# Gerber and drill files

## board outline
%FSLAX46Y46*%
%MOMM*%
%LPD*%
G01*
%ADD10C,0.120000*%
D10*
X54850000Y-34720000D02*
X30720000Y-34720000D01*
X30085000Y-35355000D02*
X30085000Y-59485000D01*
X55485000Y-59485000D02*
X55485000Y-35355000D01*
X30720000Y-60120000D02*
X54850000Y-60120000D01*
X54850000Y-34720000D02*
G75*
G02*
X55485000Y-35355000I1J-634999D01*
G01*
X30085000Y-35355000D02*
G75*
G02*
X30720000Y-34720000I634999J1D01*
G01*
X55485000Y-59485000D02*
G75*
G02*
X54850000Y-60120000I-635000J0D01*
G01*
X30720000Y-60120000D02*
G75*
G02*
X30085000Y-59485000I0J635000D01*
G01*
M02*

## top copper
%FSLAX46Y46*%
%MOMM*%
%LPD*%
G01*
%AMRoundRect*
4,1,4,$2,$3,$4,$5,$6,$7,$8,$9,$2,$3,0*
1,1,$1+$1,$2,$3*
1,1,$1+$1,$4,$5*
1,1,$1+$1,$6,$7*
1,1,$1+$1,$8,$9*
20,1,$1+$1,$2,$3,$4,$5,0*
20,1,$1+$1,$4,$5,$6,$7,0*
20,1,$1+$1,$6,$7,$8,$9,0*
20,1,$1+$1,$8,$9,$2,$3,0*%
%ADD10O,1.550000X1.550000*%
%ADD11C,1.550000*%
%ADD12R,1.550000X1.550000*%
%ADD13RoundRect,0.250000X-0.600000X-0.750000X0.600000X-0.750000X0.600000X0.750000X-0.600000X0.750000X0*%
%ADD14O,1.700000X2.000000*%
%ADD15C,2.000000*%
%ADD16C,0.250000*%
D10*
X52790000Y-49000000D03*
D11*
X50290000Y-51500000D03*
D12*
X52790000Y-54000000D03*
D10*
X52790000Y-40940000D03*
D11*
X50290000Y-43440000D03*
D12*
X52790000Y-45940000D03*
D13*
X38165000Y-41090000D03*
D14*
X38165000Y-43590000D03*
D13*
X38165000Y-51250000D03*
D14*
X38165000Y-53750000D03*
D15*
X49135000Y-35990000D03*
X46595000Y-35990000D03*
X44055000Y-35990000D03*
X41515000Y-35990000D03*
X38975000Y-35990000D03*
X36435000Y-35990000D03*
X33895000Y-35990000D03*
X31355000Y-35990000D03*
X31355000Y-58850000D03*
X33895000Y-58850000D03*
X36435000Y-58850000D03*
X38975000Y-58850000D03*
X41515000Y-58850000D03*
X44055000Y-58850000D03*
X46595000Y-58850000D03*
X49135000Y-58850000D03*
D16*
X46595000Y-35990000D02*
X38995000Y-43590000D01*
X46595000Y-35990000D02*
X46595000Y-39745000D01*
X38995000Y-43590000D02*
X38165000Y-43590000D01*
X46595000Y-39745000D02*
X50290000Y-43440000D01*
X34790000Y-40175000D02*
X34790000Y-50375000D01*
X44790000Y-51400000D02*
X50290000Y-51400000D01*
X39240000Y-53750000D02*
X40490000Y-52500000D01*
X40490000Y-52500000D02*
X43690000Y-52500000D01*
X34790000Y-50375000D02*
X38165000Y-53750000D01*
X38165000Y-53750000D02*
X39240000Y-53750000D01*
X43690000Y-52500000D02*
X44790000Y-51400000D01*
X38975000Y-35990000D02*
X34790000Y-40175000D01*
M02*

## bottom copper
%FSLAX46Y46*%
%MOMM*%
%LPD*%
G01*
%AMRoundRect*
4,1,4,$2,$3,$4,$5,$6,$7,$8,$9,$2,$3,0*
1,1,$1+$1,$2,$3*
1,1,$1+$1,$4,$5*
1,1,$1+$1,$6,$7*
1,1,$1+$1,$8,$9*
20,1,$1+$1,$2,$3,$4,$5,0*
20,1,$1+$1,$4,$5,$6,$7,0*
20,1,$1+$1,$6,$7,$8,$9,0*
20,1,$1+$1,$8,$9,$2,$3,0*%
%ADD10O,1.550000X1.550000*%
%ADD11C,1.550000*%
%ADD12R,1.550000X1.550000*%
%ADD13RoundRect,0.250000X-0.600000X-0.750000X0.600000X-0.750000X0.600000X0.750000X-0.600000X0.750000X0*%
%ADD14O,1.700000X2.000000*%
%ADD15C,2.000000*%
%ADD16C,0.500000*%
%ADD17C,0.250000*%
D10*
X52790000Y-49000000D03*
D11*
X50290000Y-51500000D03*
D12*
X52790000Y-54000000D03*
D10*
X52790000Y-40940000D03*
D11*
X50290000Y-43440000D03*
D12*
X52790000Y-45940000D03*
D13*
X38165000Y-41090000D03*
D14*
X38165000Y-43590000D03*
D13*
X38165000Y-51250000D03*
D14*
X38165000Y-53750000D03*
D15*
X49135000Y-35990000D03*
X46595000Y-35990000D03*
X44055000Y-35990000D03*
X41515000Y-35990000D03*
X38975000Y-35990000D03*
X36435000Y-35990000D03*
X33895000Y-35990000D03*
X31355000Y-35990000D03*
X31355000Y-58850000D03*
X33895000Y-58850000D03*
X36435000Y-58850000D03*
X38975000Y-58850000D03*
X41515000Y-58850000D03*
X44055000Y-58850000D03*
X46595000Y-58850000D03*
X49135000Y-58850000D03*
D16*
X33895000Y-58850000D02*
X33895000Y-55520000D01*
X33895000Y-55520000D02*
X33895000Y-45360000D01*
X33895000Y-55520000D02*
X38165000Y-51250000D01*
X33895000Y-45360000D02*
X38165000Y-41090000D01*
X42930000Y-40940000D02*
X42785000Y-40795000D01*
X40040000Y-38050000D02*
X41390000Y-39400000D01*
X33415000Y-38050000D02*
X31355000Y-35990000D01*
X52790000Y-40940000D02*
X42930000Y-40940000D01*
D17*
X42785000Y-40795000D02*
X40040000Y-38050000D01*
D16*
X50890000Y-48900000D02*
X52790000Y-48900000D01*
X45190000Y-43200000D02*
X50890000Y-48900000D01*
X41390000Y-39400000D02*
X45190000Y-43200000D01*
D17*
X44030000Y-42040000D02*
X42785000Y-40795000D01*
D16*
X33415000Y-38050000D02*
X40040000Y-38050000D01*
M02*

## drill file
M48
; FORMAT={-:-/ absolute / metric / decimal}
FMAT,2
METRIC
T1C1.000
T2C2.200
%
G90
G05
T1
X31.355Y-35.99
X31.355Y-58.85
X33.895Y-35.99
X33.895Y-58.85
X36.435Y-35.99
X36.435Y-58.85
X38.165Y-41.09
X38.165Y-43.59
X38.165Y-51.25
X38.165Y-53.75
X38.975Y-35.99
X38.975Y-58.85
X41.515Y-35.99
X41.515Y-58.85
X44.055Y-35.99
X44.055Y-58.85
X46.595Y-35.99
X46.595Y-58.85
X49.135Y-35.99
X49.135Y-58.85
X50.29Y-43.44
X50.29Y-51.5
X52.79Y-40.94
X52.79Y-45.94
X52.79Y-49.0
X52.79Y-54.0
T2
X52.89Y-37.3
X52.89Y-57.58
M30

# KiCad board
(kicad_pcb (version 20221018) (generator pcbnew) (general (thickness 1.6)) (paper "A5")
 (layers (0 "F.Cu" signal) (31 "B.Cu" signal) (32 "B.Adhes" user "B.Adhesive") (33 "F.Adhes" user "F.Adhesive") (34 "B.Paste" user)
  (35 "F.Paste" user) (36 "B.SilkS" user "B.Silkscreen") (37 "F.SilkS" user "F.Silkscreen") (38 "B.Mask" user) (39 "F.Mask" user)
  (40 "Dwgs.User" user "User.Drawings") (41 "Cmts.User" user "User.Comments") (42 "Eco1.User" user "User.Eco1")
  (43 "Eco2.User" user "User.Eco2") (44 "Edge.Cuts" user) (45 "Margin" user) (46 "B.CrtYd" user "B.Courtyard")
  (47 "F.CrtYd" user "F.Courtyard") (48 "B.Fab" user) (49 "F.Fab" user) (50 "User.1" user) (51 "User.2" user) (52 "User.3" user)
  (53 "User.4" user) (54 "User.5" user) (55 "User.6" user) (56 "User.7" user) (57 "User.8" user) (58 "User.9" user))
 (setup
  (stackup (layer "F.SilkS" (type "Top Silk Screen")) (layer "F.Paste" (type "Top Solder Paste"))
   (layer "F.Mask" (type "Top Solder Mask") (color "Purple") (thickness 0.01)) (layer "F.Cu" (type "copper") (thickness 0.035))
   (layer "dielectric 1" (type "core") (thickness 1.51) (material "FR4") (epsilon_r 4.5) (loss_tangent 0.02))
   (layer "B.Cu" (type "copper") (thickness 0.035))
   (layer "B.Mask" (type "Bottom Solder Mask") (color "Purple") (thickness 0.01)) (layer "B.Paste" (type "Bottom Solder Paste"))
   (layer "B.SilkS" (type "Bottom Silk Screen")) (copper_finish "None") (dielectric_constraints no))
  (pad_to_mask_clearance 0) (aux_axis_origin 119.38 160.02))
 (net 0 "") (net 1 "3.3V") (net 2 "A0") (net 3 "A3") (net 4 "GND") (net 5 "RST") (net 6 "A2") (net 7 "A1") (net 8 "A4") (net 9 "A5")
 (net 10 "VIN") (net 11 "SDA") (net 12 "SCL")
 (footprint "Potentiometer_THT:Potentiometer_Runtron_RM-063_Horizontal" (layer "F.Cu") (at 52.79 49 -90)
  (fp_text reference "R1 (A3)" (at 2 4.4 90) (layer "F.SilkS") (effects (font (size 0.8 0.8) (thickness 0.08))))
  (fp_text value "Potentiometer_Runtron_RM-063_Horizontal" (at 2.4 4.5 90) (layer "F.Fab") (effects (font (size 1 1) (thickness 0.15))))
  (pad "1" thru_hole oval (at 0 0 270) (size 1.55 1.55) (drill 1) (layers "*.Cu" "*.Mask") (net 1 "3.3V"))
  (pad "2" thru_hole circle (at 2.5 2.5 270) (size 1.55 1.55) (drill 1) (layers "*.Cu" "*.Mask") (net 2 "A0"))
  (pad "3" thru_hole rect (at 5 0 270) (size 1.55 1.55) (drill 1) (layers "*.Cu" "*.Mask")))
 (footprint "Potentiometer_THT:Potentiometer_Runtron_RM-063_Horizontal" (layer "F.Cu") (at 52.79 40.94 -90)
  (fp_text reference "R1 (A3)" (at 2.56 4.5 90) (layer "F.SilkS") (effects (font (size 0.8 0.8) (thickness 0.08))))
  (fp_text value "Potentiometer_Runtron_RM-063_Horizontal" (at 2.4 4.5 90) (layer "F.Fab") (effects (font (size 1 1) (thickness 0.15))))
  (pad "1" thru_hole oval (at 0 0 270) (size 1.55 1.55) (drill 1) (layers "*.Cu" "*.Mask") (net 1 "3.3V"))
  (pad "2" thru_hole circle (at 2.5 2.5 270) (size 1.55 1.55) (drill 1) (layers "*.Cu" "*.Mask") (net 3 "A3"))
  (pad "3" thru_hole rect (at 5 0 270) (size 1.55 1.55) (drill 1) (layers "*.Cu" "*.Mask")))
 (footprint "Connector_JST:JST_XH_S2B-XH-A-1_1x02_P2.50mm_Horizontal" (layer "F.Cu") (at 30.065 42.34 -90)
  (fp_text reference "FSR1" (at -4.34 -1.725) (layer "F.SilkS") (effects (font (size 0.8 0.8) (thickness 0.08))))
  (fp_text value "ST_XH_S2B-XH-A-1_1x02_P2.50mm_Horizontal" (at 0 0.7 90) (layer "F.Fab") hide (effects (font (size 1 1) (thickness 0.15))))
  (pad "1" thru_hole roundrect (at -1.25 -8.1) (size 1.7 2) (drill 1) (layers "*.Cu" "*.Mask") (roundrect_rratio 0.1470588235) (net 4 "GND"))
  (pad "2" thru_hole oval (at 1.25 -8.1) (size 1.7 2) (drill 1) (layers "*.Cu" "*.Mask") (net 3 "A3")))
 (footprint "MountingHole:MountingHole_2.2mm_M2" (layer "F.Cu") (at 52.89 57.54)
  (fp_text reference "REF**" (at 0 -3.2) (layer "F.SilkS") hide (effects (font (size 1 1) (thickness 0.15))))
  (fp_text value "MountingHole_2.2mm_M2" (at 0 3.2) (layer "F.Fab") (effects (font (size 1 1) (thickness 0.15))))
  (pad "" np_thru_hole circle (at 0 0.04) (size 2.2 2.2) (drill 2.2) (layers "*.Cu" "*.Mask")))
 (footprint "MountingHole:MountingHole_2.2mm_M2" (layer "F.Cu") (at 52.89 37.3)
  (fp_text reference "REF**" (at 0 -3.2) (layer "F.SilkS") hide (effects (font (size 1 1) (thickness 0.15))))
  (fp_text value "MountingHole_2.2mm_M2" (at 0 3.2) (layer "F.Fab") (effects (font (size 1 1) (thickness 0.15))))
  (pad "" np_thru_hole circle (at 0 0) (size 2.2 2.2) (drill 2.2) (layers "*.Cu" "*.Mask")))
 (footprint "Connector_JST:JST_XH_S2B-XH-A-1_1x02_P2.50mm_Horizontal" (layer "F.Cu") (at 30.065 52.5 -90)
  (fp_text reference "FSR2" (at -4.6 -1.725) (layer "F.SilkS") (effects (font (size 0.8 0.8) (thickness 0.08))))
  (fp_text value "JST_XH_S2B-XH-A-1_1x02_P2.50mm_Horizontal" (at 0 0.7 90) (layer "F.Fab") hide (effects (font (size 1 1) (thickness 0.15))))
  (pad "1" thru_hole roundrect (at -1.25 -8.1) (size 1.7 2) (drill 1) (layers "*.Cu" "*.Mask") (roundrect_rratio 0.1470588235) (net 4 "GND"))
  (pad "2" thru_hole oval (at 1.25 -8.1) (size 1.7 2) (drill 1) (layers "*.Cu" "*.Mask") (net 2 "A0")))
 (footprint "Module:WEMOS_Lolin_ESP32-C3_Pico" (layer "F.Cu") (at 30.085 47.42 -90)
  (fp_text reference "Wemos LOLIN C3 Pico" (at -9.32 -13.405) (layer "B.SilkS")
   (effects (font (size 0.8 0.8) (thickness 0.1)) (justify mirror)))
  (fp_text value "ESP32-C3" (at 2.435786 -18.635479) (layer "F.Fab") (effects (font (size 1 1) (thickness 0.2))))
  (fp_line (start -12.7 -24.765) (end -12.7 -0.635) (stroke (width 0.12) (type solid)) (layer "Edge.Cuts"))
  (fp_line (start -12.065 0) (end 12.065 0) (stroke (width 0.12) (type solid)) (layer "Edge.Cuts"))
  (fp_line (start 12.065 -25.4) (end -12.065 -25.4) (stroke (width 0.12) (type solid)) (layer "Edge.Cuts"))
  (fp_line (start 12.7 -0.635) (end 12.7 -24.765) (stroke (width 0.12) (type solid)) (layer "Edge.Cuts"))
  (fp_arc (start -12.7 -24.765) (mid -12.514013 -25.214013) (end -12.065 -25.4) (stroke (width 0.12) (type solid)) (layer "Edge.Cuts"))
  (fp_arc (start -12.065 0) (mid -12.514013 -0.185987) (end -12.7 -0.635) (stroke (width 0.12) (type solid)) (layer "Edge.Cuts"))
  (fp_arc (start 12.065 -25.4) (mid 12.514013 -25.214013) (end 12.7 -24.765) (stroke (width 0.12) (type solid)) (layer "Edge.Cuts"))
  (fp_arc (start 12.7 -0.635) (mid 12.514013 -0.185987) (end 12.065 0) (stroke (width 0.12) (type solid)) (layer "Edge.Cuts"))
  (pad "1" thru_hole circle (at -11.43 -19.05 270) (size 2 2) (drill 1) (layers "*.Cu" "*.Mask") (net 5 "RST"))
  (pad "2" thru_hole circle (at -11.43 -16.51 270) (size 2 2) (drill 1) (layers "*.Cu" "*.Mask") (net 3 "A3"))
  (pad "3" thru_hole circle (at -11.43 -13.97 270) (size 2 2) (drill 1) (layers "*.Cu" "*.Mask") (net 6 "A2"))
  (pad "4" thru_hole circle (at -11.43 -11.43 270) (size 2 2) (drill 1) (layers "*.Cu" "*.Mask") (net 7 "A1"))
  (pad "5" thru_hole circle (at -11.43 -8.89 270) (size 2 2) (drill 1) (layers "*.Cu" "*.Mask") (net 2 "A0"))
  (pad "6" thru_hole circle (at -11.43 -6.35 270) (size 2 2) (drill 1) (layers "*.Cu" "*.Mask") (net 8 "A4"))
  (pad "7" thru_hole circle (at -11.43 -3.81 270) (size 2 2) (drill 1) (layers "*.Cu" "*.Mask") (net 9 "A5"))
  (pad "8" thru_hole circle (at -11.43 -1.27 270) (size 2 2) (drill 1) (layers "*.Cu" "*.Mask") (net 1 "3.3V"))
  (pad "9" thru_hole circle (at 11.43 -1.27 270) (size 2 2) (drill 1) (layers "*.Cu" "*.Mask") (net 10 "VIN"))
  (pad "10" thru_hole circle (at 11.43 -3.81 270) (size 2 2) (drill 1) (layers "*.Cu" "*.Mask") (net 4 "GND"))
  (pad "11" thru_hole circle (at 11.43 -6.35 270) (size 2 2) (drill 1) (layers "*.Cu" "*.Mask"))
  (pad "12" thru_hole circle (at 11.43 -8.89 270) (size 2 2) (drill 1) (layers "*.Cu" "*.Mask"))
  (pad "13" thru_hole circle (at 11.43 -11.43 270) (size 2 2) (drill 1) (layers "*.Cu" "*.Mask") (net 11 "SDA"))
  (pad "14" thru_hole circle (at 11.43 -13.97 270) (size 2 2) (drill 1) (layers "*.Cu" "*.Mask") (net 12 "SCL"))
  (pad "15" thru_hole circle (at 11.43 -16.51 270) (size 2 2) (drill 1) (layers "*.Cu" "*.Mask"))
  (pad "16" thru_hole circle (at 11.43 -19.05 270) (size 2 2) (drill 1) (layers "*.Cu" "*.Mask")))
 (segment (start 33.895 58.85) (end 33.895 55.52) (width 0.5) (layer "B.Cu") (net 4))
 (segment (start 33.895 55.52) (end 33.895 45.36) (width 0.5) (layer "B.Cu") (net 4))
 (segment (start 33.895 55.52) (end 38.165 51.25) (width 0.5) (layer "B.Cu") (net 4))
 (segment (start 33.895 45.36) (end 38.165 41.09) (width 0.5) (layer "B.Cu") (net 4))
 (segment (start 42.93 40.94) (end 42.785 40.795) (width 0.5) (layer "B.Cu") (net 1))
 (segment (start 40.04 38.05) (end 41.39 39.4) (width 0.5) (layer "B.Cu") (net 1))
 (segment (start 33.415 38.05) (end 31.355 35.99) (width 0.5) (layer "B.Cu") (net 1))
 (segment (start 52.79 40.94) (end 42.93 40.94) (width 0.5) (layer "B.Cu") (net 1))
 (segment (start 42.785 40.795) (end 40.04 38.05) (width 0.25) (layer "B.Cu") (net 1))
 (segment (start 50.89 48.9) (end 52.79 48.9) (width 0.5) (layer "B.Cu") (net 1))
 (segment (start 45.19 43.2) (end 50.89 48.9) (width 0.5) (layer "B.Cu") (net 1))
 (segment (start 41.39 39.4) (end 45.19 43.2) (width 0.5) (layer "B.Cu") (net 1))
 (segment (start 44.03 42.04) (end 42.785 40.795) (width 0.25) (layer "B.Cu") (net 1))
 (segment (start 33.415 38.05) (end 40.04 38.05) (width 0.5) (layer "B.Cu") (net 1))
 (segment (start 46.595 35.99) (end 38.995 43.59) (width 0.25) (layer "F.Cu") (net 3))
 (segment (start 46.595 35.99) (end 46.595 39.745) (width 0.25) (layer "F.Cu") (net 3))
 (segment (start 38.995 43.59) (end 38.165 43.59) (width 0.25) (layer "F.Cu") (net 3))
 (segment (start 46.595 39.745) (end 50.29 43.44) (width 0.25) (layer "F.Cu") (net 3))
 (segment (start 34.79 40.175) (end 34.79 50.375) (width 0.25) (layer "F.Cu") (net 2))
 (segment (start 44.79 51.4) (end 50.29 51.4) (width 0.25) (layer "F.Cu") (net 2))
 (segment (start 39.24 53.75) (end 40.49 52.5) (width 0.25) (layer "F.Cu") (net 2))
 (segment (start 40.49 52.5) (end 43.69 52.5) (width 0.25) (layer "F.Cu") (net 2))
 (segment (start 34.79 50.375) (end 38.165 53.75) (width 0.25) (layer "F.Cu") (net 2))
 (segment (start 38.165 53.75) (end 39.24 53.75) (width 0.25) (layer "F.Cu") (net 2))
 (segment (start 43.69 52.5) (end 44.79 51.4) (width 0.25) (layer "F.Cu") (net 2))
 (segment (start 38.975 35.99) (end 34.79 40.175) (width 0.25) (layer "F.Cu") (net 2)))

